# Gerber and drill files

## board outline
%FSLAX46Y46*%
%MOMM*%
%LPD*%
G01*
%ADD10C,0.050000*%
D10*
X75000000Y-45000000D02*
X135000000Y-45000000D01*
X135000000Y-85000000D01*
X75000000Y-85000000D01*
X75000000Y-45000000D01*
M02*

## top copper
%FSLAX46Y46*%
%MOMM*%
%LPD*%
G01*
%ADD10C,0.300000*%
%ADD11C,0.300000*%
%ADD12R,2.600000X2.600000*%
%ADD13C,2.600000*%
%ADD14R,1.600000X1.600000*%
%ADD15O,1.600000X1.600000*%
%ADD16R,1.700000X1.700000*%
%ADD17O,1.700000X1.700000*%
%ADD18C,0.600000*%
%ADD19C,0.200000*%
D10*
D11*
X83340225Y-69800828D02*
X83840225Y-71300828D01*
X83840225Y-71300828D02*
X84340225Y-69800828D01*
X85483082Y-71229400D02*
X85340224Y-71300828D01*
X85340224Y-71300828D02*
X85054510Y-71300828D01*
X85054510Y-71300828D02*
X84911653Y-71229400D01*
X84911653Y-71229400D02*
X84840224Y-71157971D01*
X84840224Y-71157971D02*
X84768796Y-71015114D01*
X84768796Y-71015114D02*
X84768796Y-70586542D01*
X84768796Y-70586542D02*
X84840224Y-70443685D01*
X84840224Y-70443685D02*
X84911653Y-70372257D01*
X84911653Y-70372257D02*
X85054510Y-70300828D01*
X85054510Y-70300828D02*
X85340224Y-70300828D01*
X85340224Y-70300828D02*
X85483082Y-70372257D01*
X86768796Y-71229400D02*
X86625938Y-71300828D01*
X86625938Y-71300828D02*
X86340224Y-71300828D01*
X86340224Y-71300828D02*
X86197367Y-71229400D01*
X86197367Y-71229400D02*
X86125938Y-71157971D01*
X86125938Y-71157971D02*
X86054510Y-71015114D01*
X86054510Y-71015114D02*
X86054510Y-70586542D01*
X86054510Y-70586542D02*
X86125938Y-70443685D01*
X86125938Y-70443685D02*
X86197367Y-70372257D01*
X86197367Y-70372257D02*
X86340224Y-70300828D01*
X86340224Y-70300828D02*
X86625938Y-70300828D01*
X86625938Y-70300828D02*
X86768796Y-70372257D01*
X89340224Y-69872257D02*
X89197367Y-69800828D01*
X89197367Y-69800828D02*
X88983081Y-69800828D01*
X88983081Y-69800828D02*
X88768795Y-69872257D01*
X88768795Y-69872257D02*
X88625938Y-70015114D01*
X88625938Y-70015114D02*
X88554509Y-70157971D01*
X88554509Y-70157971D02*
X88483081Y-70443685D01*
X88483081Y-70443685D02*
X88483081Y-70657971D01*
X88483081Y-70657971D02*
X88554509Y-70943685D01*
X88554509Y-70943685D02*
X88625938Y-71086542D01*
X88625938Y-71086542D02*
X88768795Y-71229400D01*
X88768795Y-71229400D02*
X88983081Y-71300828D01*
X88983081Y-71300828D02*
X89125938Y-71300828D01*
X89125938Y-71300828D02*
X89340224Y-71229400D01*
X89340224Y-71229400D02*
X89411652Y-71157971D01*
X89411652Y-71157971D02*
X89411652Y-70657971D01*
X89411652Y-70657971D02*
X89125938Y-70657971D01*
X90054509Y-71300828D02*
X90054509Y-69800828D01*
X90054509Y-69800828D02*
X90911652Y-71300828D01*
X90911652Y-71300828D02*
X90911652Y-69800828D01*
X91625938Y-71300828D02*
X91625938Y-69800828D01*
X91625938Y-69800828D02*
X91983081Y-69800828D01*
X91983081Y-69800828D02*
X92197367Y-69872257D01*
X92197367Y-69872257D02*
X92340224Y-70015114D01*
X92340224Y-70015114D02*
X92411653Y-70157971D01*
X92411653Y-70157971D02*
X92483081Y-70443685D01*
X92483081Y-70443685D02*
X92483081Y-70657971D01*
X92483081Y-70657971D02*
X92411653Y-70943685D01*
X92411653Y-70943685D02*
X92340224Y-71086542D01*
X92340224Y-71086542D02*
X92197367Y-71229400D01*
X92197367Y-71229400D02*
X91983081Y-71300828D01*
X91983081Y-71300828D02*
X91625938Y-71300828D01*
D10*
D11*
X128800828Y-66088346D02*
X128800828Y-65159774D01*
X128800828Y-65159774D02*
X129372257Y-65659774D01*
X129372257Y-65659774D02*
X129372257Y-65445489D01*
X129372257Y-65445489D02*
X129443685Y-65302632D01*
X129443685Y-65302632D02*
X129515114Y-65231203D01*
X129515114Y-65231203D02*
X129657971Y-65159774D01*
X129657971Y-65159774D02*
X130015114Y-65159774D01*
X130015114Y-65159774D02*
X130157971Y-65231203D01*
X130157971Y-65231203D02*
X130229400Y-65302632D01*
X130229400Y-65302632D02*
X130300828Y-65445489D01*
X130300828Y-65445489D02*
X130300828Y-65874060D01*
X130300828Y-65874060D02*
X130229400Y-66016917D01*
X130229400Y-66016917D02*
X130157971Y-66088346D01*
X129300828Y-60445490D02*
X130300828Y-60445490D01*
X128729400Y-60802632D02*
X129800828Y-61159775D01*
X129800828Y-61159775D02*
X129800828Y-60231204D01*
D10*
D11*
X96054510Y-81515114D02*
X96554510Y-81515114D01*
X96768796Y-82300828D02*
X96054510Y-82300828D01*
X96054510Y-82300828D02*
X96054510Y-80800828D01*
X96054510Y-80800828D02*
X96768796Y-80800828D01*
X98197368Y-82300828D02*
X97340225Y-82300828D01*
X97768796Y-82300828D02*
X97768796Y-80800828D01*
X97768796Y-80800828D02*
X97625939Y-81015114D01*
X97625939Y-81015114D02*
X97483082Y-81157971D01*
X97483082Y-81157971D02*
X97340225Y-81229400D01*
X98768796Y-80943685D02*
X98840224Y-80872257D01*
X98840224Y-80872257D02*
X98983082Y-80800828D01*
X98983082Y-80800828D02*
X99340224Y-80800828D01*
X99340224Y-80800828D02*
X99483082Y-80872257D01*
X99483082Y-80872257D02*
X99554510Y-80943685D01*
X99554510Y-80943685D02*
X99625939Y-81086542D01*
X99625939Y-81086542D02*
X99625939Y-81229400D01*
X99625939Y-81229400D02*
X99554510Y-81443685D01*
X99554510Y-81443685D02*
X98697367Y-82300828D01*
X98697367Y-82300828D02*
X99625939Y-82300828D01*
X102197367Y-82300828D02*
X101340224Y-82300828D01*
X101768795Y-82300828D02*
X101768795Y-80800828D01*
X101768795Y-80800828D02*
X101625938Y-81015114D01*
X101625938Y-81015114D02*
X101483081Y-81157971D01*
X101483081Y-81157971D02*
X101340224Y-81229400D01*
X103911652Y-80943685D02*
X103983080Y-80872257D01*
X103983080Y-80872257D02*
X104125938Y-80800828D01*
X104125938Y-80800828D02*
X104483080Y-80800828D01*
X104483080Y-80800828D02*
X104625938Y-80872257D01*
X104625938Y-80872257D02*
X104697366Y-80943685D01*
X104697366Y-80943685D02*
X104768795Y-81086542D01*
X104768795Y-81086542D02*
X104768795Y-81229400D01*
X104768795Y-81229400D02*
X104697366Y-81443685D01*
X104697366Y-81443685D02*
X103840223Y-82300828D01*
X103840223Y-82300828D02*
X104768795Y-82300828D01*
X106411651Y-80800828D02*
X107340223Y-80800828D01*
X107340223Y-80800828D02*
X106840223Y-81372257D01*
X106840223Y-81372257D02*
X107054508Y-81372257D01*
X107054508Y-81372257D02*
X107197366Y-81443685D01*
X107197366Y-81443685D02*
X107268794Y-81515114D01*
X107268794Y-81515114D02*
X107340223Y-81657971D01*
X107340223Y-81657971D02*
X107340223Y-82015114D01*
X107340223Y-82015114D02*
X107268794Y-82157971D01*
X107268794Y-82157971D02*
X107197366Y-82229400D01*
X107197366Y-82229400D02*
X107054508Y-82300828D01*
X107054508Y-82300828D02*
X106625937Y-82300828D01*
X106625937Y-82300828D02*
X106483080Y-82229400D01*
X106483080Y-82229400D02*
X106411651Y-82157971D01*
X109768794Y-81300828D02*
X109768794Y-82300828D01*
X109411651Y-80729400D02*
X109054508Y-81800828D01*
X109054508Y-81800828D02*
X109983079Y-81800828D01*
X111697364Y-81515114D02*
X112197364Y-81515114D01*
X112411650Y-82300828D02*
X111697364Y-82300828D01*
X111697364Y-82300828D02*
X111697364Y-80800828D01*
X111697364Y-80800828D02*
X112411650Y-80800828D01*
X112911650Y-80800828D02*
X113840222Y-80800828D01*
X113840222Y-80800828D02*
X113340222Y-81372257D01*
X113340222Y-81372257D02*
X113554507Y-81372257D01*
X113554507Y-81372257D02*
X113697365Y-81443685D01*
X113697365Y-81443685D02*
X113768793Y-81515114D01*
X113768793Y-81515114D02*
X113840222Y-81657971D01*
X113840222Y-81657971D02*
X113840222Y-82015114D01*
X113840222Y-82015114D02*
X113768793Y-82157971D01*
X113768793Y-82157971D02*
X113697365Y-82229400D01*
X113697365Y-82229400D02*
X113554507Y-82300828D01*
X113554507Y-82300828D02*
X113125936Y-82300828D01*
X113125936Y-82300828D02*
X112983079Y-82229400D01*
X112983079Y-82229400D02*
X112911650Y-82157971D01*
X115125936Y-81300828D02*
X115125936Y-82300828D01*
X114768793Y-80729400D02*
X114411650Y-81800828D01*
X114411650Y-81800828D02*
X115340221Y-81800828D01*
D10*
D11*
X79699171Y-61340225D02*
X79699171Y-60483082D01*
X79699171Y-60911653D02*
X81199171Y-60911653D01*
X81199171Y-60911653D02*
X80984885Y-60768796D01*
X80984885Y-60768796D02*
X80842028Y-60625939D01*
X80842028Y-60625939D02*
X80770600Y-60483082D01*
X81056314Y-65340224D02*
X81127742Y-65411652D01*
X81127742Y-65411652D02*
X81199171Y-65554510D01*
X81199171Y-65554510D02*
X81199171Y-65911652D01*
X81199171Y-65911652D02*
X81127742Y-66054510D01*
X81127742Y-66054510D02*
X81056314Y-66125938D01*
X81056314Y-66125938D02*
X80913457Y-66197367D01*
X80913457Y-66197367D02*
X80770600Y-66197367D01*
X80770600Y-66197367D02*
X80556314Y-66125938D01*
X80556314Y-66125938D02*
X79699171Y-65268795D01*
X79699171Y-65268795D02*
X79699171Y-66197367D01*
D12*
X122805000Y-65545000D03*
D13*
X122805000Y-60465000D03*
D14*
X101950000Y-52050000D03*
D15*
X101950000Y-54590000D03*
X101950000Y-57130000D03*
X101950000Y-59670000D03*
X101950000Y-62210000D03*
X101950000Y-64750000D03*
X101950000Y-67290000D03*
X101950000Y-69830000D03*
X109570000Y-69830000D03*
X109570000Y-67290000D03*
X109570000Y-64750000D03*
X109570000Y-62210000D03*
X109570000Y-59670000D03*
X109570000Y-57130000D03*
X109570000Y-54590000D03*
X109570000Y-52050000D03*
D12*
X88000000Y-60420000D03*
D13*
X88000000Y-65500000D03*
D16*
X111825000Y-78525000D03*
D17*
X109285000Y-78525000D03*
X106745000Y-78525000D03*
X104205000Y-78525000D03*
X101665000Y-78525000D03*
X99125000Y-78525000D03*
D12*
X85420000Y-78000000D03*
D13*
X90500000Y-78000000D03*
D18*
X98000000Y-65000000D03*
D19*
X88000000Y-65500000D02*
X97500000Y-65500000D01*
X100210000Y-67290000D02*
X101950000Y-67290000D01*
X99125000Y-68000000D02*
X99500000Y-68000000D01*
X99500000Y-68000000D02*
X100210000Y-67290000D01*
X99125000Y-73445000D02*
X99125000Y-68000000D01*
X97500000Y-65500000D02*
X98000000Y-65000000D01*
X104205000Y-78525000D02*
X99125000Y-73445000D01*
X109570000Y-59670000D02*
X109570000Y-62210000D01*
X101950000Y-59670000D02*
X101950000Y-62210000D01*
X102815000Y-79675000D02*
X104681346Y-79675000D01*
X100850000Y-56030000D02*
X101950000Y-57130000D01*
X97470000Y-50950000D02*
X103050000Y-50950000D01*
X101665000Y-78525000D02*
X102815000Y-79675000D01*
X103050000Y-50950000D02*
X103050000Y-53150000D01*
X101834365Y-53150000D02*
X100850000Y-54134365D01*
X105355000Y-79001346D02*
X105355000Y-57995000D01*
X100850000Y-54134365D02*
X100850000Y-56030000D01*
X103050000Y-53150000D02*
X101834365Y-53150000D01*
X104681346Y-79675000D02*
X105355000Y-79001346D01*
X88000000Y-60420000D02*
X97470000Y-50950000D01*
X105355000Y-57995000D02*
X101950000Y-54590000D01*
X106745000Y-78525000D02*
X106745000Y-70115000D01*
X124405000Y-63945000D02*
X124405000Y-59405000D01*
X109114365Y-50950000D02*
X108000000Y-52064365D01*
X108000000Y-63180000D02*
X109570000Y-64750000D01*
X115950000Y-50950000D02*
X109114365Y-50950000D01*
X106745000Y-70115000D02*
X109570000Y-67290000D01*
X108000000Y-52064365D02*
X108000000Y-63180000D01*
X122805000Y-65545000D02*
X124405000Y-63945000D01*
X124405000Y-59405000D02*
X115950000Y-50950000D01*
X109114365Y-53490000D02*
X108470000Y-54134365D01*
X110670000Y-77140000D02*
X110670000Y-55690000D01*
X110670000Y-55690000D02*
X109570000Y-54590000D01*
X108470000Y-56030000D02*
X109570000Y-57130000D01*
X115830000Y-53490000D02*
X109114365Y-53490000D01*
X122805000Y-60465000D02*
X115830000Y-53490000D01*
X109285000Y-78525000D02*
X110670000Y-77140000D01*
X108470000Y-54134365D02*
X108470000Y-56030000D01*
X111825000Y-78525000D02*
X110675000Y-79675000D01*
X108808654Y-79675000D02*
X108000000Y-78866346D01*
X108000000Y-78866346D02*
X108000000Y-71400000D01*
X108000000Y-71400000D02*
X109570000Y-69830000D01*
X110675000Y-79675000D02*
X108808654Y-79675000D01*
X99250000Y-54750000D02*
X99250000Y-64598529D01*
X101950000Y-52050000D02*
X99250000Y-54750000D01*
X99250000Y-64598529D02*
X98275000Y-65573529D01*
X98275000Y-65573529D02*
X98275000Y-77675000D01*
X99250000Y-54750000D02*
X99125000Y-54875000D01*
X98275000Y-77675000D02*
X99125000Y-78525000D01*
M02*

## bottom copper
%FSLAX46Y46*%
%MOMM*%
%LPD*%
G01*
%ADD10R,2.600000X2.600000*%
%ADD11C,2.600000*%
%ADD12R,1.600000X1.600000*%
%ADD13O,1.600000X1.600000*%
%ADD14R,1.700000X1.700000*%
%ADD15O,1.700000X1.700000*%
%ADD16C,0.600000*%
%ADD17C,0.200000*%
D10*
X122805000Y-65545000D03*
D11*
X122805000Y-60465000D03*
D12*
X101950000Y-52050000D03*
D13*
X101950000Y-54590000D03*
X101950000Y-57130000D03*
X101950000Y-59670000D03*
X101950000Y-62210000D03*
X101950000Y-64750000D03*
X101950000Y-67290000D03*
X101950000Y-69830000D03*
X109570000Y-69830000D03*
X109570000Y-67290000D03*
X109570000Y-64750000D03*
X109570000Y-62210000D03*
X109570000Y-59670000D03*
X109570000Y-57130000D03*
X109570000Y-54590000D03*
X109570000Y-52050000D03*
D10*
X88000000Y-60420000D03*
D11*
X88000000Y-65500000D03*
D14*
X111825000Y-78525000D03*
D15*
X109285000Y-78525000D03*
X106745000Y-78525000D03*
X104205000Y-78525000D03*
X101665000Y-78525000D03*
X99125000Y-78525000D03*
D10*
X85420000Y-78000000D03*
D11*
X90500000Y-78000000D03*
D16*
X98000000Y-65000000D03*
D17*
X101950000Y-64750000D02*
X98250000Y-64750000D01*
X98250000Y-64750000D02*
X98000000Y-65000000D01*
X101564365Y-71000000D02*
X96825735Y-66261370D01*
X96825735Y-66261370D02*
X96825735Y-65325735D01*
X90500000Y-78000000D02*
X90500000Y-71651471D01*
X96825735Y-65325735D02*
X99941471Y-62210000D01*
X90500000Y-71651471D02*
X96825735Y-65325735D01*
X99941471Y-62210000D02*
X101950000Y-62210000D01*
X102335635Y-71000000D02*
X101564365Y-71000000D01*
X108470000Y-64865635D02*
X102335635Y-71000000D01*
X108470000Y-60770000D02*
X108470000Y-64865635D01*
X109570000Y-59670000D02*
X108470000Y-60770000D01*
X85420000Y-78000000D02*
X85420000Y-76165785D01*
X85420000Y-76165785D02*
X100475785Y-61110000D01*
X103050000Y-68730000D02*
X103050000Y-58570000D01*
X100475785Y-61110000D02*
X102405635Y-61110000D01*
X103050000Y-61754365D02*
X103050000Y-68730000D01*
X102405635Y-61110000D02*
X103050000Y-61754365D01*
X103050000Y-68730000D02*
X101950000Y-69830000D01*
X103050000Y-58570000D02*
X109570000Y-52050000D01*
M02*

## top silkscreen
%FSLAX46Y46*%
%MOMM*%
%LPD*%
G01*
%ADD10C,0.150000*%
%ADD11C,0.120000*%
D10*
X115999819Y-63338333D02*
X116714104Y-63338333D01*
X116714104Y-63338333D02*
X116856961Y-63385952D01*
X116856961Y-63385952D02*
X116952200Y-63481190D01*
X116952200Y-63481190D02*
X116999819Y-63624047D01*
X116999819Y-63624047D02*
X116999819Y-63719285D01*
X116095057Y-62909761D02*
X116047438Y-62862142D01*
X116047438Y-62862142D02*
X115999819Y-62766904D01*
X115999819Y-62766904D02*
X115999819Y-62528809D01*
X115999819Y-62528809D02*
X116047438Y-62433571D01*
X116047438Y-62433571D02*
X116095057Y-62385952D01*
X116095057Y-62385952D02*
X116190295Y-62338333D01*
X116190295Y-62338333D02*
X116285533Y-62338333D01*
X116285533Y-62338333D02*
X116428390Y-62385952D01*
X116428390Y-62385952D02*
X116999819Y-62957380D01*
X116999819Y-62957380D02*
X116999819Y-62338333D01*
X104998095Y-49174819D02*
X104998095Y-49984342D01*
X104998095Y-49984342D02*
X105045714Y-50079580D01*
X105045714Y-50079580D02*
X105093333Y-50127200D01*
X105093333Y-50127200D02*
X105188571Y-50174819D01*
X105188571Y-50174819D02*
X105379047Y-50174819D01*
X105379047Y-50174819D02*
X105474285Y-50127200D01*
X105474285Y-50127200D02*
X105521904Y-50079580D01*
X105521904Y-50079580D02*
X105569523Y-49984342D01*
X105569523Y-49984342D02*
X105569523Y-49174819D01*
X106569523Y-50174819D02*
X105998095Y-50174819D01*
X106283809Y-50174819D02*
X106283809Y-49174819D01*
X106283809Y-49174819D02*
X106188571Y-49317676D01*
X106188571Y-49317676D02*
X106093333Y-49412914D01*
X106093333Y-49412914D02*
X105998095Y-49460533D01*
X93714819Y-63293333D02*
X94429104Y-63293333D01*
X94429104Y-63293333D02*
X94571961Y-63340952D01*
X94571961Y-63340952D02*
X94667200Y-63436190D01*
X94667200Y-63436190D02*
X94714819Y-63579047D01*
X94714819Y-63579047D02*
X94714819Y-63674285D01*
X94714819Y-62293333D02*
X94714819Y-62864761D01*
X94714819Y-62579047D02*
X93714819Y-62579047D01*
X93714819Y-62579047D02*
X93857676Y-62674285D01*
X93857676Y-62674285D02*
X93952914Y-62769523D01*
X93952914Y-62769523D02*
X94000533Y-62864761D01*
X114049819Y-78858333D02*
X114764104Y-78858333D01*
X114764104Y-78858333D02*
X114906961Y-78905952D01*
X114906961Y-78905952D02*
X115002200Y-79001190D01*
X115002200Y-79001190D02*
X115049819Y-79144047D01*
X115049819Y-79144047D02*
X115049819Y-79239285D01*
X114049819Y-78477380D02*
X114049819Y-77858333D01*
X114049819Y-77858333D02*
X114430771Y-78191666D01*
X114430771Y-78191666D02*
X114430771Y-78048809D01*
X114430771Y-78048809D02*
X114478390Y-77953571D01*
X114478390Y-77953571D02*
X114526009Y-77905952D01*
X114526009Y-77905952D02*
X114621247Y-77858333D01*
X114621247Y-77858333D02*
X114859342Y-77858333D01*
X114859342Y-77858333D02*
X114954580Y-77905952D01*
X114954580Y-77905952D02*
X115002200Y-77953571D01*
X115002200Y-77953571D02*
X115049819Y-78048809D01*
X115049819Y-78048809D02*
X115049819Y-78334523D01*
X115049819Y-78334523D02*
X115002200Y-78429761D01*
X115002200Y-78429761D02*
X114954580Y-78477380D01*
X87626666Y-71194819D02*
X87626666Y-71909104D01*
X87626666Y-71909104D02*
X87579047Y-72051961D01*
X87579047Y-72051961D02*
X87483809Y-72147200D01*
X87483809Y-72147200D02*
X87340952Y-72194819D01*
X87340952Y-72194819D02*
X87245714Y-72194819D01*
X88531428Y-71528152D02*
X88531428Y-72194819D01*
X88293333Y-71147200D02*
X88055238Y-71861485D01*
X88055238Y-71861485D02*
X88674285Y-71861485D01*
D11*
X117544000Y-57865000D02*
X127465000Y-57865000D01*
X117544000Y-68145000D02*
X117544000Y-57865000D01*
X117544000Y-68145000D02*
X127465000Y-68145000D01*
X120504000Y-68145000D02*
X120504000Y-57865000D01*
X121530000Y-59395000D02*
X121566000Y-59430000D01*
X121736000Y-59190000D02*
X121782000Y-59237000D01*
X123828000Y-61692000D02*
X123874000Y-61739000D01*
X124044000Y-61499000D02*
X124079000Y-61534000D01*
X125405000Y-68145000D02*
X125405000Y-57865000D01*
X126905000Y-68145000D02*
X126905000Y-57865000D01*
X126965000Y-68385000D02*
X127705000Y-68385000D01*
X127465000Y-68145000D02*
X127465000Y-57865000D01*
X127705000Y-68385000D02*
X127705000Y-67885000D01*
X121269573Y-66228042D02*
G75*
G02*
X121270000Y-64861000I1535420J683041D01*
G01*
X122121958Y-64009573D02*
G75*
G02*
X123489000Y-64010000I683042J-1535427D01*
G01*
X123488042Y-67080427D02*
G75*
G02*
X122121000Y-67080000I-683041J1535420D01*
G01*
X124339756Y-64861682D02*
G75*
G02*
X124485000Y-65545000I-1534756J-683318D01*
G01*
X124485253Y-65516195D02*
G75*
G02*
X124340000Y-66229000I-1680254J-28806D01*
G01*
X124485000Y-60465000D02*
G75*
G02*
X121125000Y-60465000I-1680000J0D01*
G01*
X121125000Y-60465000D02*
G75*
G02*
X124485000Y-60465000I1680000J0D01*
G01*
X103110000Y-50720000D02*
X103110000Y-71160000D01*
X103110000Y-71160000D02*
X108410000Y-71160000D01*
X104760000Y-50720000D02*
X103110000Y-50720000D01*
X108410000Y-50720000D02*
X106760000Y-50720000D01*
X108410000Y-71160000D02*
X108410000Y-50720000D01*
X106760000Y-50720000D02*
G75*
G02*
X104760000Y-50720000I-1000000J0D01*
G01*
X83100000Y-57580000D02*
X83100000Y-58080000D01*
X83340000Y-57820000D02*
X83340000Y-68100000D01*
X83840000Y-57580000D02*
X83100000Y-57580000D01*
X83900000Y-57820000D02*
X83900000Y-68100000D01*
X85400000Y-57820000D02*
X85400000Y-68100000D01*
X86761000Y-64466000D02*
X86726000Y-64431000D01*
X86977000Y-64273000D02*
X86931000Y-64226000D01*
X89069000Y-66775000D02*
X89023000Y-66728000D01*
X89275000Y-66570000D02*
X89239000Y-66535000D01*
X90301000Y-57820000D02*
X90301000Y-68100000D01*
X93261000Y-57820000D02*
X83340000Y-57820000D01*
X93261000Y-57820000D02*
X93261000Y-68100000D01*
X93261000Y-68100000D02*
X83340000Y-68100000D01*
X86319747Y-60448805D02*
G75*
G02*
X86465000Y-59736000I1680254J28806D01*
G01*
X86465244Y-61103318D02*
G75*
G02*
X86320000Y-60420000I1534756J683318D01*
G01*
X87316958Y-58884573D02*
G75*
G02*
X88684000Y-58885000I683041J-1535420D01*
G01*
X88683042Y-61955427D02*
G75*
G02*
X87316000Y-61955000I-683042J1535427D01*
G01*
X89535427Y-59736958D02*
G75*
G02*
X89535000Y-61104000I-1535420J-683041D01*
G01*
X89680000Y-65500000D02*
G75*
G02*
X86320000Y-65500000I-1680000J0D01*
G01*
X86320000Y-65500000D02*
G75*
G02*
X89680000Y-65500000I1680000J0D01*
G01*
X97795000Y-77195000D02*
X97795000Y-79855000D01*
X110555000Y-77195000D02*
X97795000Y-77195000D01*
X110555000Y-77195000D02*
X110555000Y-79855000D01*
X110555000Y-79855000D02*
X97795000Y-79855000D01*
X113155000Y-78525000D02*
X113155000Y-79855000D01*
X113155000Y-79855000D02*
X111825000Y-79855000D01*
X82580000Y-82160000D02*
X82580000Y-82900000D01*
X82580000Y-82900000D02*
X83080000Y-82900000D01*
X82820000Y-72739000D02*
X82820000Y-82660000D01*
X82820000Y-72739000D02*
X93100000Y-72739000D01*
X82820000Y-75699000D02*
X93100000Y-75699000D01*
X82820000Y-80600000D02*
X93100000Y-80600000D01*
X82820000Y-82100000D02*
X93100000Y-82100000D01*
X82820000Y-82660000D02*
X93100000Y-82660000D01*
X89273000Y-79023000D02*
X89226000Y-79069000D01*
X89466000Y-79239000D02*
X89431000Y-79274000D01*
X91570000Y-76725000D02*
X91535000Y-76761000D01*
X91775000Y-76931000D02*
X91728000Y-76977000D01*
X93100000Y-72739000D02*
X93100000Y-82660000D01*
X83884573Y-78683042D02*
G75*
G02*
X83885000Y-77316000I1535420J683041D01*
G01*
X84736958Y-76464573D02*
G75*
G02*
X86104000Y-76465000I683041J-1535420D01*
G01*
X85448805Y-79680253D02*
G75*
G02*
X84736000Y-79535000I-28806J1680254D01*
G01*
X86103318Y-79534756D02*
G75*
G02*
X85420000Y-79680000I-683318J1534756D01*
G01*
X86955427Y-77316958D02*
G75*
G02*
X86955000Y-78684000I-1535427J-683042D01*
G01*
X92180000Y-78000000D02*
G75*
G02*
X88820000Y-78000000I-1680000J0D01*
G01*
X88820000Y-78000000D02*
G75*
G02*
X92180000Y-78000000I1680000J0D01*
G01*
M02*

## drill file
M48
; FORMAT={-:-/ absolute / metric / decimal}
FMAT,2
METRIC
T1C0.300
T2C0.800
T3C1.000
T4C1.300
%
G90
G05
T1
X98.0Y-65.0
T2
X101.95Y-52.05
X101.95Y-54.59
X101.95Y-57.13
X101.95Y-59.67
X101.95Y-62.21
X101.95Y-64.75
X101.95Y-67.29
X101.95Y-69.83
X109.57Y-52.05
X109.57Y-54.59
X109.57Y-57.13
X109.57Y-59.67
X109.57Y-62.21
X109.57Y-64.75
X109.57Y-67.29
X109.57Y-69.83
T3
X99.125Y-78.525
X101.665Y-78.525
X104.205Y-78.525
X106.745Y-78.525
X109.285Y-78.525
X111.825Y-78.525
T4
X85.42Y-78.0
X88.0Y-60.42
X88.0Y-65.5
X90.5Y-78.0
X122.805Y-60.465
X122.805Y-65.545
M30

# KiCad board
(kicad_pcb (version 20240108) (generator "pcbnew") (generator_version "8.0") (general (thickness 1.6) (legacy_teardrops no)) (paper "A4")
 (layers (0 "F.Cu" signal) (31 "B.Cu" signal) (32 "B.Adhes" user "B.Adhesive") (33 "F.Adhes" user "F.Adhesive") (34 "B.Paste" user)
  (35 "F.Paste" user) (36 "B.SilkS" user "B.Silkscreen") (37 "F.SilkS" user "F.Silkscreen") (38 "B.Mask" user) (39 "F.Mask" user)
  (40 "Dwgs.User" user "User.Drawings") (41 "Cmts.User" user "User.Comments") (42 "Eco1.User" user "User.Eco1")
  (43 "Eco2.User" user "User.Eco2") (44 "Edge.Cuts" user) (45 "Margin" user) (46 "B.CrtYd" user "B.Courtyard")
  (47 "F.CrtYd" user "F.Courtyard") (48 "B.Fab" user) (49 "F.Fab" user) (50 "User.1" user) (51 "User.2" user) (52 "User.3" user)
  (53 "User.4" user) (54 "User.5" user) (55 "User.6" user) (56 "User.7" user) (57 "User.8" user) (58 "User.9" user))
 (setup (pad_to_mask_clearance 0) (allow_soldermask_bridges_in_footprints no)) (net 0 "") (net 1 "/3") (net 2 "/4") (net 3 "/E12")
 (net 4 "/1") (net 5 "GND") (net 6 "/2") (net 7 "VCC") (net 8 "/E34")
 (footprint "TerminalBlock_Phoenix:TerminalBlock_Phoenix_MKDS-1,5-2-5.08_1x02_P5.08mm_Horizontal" (layer "F.Cu") (at 122.805 65.545 90)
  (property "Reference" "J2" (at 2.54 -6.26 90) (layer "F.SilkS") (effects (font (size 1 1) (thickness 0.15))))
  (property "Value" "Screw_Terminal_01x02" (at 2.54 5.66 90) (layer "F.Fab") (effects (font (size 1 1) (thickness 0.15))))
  (fp_line (start 7.68 -5.261) (end 7.68 4.66) (stroke (width 0.12) (type solid)) (layer "F.SilkS"))
  (fp_line (start -2.6 -5.261) (end 7.68 -5.261) (stroke (width 0.12) (type solid)) (layer "F.SilkS"))
  (fp_line (start -2.6 -5.261) (end -2.6 4.66) (stroke (width 0.12) (type solid)) (layer "F.SilkS"))
  (fp_line (start -2.6 -2.301) (end 7.68 -2.301) (stroke (width 0.12) (type solid)) (layer "F.SilkS"))
  (fp_line (start 6.15 -1.275) (end 6.115 -1.239) (stroke (width 0.12) (type solid)) (layer "F.SilkS"))
  (fp_line (start 6.355 -1.069) (end 6.308 -1.023) (stroke (width 0.12) (type solid)) (layer "F.SilkS"))
  (fp_line (start 3.853 1.023) (end 3.806 1.069) (stroke (width 0.12) (type solid)) (layer "F.SilkS"))
  (fp_line (start 4.046 1.239) (end 4.011 1.274) (stroke (width 0.12) (type solid)) (layer "F.SilkS"))
  (fp_line (start -2.6 2.6) (end 7.68 2.6) (stroke (width 0.12) (type solid)) (layer "F.SilkS"))
  (fp_line (start -2.6 4.1) (end 7.68 4.1) (stroke (width 0.12) (type solid)) (layer "F.SilkS"))
  (fp_line (start -2.84 4.16) (end -2.84 4.9) (stroke (width 0.12) (type solid)) (layer "F.SilkS"))
  (fp_line (start -2.6 4.66) (end 7.68 4.66) (stroke (width 0.12) (type solid)) (layer "F.SilkS"))
  (fp_line (start -2.84 4.9) (end -2.34 4.9) (stroke (width 0.12) (type solid)) (layer "F.SilkS"))
  (fp_arc (start -0.683042 -1.535427) (mid 0.000524 -1.680501) (end 0.684 -1.535) (stroke (width 0.12) (type solid)) (layer "F.SilkS"))
  (fp_arc (start 1.535427 -0.683042) (mid 1.680501 0.000524) (end 1.535 0.684) (stroke (width 0.12) (type solid)) (layer "F.SilkS"))
  (fp_arc (start -1.535427 0.683042) (mid -1.680501 -0.000524) (end -1.535 -0.684) (stroke (width 0.12) (type solid)) (layer "F.SilkS"))
  (fp_arc (start 0.683318 1.534756) (mid 0.349292 1.643288) (end 0 1.68) (stroke (width 0.12) (type solid)) (layer "F.SilkS"))
  (fp_arc (start 0.028805 1.680253) (mid -0.335551 1.646659) (end -0.684 1.535) (stroke (width 0.12) (type solid)) (layer "F.SilkS"))
  (fp_circle (center 5.08 0) (end 6.76 0) (stroke (width 0.12) (type solid)) (fill none) (layer "F.SilkS"))
  (pad "1" thru_hole rect (at 0 0 90) (size 2.6 2.6) (drill 1.3) (layers "*.Cu" "*.Mask") (remove_unused_layers no) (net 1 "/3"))
  (pad "2" thru_hole circle (at 5.08 0 90) (size 2.6 2.6) (drill 1.3) (layers "*.Cu" "*.Mask") (remove_unused_layers no) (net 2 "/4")))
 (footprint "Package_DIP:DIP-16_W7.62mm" (layer "F.Cu") (at 101.95 52.05)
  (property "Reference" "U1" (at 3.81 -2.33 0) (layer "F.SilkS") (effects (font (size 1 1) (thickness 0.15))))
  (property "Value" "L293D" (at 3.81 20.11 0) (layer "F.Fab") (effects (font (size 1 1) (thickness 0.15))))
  (fp_line (start 1.16 -1.33) (end 1.16 19.11) (stroke (width 0.12) (type solid)) (layer "F.SilkS"))
  (fp_line (start 1.16 19.11) (end 6.46 19.11) (stroke (width 0.12) (type solid)) (layer "F.SilkS"))
  (fp_line (start 2.81 -1.33) (end 1.16 -1.33) (stroke (width 0.12) (type solid)) (layer "F.SilkS"))
  (fp_line (start 6.46 -1.33) (end 4.81 -1.33) (stroke (width 0.12) (type solid)) (layer "F.SilkS"))
  (fp_line (start 6.46 19.11) (end 6.46 -1.33) (stroke (width 0.12) (type solid)) (layer "F.SilkS"))
  (fp_arc (start 4.81 -1.33) (mid 3.81 -0.33) (end 2.81 -1.33) (stroke (width 0.12) (type solid)) (layer "F.SilkS"))
  (pad "1" thru_hole rect (at 0 0) (size 1.6 1.6) (drill 0.8) (layers "*.Cu" "*.Mask") (remove_unused_layers no) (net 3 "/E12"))
  (pad "2" thru_hole oval (at 0 2.54) (size 1.6 1.6) (drill 0.8) (layers "*.Cu" "*.Mask") (remove_unused_layers no) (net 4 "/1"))
  (pad "3" thru_hole oval (at 0 5.08) (size 1.6 1.6) (drill 0.8) (layers "*.Cu" "*.Mask") (remove_unused_layers no) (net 4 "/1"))
  (pad "4" thru_hole oval (at 0 7.62) (size 1.6 1.6) (drill 0.8) (layers "*.Cu" "*.Mask") (remove_unused_layers no) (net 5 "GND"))
  (pad "5" thru_hole oval (at 0 10.16) (size 1.6 1.6) (drill 0.8) (layers "*.Cu" "*.Mask") (remove_unused_layers no) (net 5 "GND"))
  (pad "6" thru_hole oval (at 0 12.7) (size 1.6 1.6) (drill 0.8) (layers "*.Cu" "*.Mask") (remove_unused_layers no) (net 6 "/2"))
  (pad "7" thru_hole oval (at 0 15.24) (size 1.6 1.6) (drill 0.8) (layers "*.Cu" "*.Mask") (remove_unused_layers no) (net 6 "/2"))
  (pad "8" thru_hole oval (at 0 17.78) (size 1.6 1.6) (drill 0.8) (layers "*.Cu" "*.Mask") (remove_unused_layers no) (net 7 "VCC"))
  (pad "9" thru_hole oval (at 7.62 17.78) (size 1.6 1.6) (drill 0.8) (layers "*.Cu" "*.Mask") (remove_unused_layers no) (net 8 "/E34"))
  (pad "10" thru_hole oval (at 7.62 15.24) (size 1.6 1.6) (drill 0.8) (layers "*.Cu" "*.Mask") (remove_unused_layers no) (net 1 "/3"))
  (pad "11" thru_hole oval (at 7.62 12.7) (size 1.6 1.6) (drill 0.8) (layers "*.Cu" "*.Mask") (remove_unused_layers no) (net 1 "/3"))
  (pad "12" thru_hole oval (at 7.62 10.16) (size 1.6 1.6) (drill 0.8) (layers "*.Cu" "*.Mask") (remove_unused_layers no) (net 5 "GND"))
  (pad "13" thru_hole oval (at 7.62 7.62) (size 1.6 1.6) (drill 0.8) (layers "*.Cu" "*.Mask") (remove_unused_layers no) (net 5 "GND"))
  (pad "14" thru_hole oval (at 7.62 5.08) (size 1.6 1.6) (drill 0.8) (layers "*.Cu" "*.Mask") (remove_unused_layers no) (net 2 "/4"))
  (pad "15" thru_hole oval (at 7.62 2.54) (size 1.6 1.6) (drill 0.8) (layers "*.Cu" "*.Mask") (remove_unused_layers no) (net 2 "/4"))
  (pad "16" thru_hole oval (at 7.62 0) (size 1.6 1.6) (drill 0.8) (layers "*.Cu" "*.Mask") (remove_unused_layers no) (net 7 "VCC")))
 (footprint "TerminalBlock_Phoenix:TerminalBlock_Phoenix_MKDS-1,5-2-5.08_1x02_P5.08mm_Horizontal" (layer "F.Cu") (at 88 60.42 -90)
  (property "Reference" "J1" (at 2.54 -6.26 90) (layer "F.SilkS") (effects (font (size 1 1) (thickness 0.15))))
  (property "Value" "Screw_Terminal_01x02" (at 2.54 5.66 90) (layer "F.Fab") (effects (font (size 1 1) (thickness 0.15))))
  (fp_line (start -2.84 4.9) (end -2.34 4.9) (stroke (width 0.12) (type solid)) (layer "F.SilkS"))
  (fp_line (start -2.6 4.66) (end 7.68 4.66) (stroke (width 0.12) (type solid)) (layer "F.SilkS"))
  (fp_line (start -2.84 4.16) (end -2.84 4.9) (stroke (width 0.12) (type solid)) (layer "F.SilkS"))
  (fp_line (start -2.6 4.1) (end 7.68 4.1) (stroke (width 0.12) (type solid)) (layer "F.SilkS"))
  (fp_line (start -2.6 2.6) (end 7.68 2.6) (stroke (width 0.12) (type solid)) (layer "F.SilkS"))
  (fp_line (start 4.046 1.239) (end 4.011 1.274) (stroke (width 0.12) (type solid)) (layer "F.SilkS"))
  (fp_line (start 3.853 1.023) (end 3.806 1.069) (stroke (width 0.12) (type solid)) (layer "F.SilkS"))
  (fp_line (start 6.355 -1.069) (end 6.308 -1.023) (stroke (width 0.12) (type solid)) (layer "F.SilkS"))
  (fp_line (start 6.15 -1.275) (end 6.115 -1.239) (stroke (width 0.12) (type solid)) (layer "F.SilkS"))
  (fp_line (start -2.6 -2.301) (end 7.68 -2.301) (stroke (width 0.12) (type solid)) (layer "F.SilkS"))
  (fp_line (start -2.6 -5.261) (end -2.6 4.66) (stroke (width 0.12) (type solid)) (layer "F.SilkS"))
  (fp_line (start -2.6 -5.261) (end 7.68 -5.261) (stroke (width 0.12) (type solid)) (layer "F.SilkS"))
  (fp_line (start 7.68 -5.261) (end 7.68 4.66) (stroke (width 0.12) (type solid)) (layer "F.SilkS"))
  (fp_arc (start 0.028805 1.680253) (mid -0.335551 1.646659) (end -0.684 1.535) (stroke (width 0.12) (type solid)) (layer "F.SilkS"))
  (fp_arc (start 0.683318 1.534756) (mid 0.349292 1.643288) (end 0 1.68) (stroke (width 0.12) (type solid)) (layer "F.SilkS"))
  (fp_arc (start -1.535427 0.683042) (mid -1.680501 -0.000524) (end -1.535 -0.684) (stroke (width 0.12) (type solid)) (layer "F.SilkS"))
  (fp_arc (start 1.535427 -0.683042) (mid 1.680501 0.000524) (end 1.535 0.684) (stroke (width 0.12) (type solid)) (layer "F.SilkS"))
  (fp_arc (start -0.683042 -1.535427) (mid 0.000524 -1.680501) (end 0.684 -1.535) (stroke (width 0.12) (type solid)) (layer "F.SilkS"))
  (fp_circle (center 5.08 0) (end 6.76 0) (stroke (width 0.12) (type solid)) (fill none) (layer "F.SilkS"))
  (pad "1" thru_hole rect (at 0 0 270) (size 2.6 2.6) (drill 1.3) (layers "*.Cu" "*.Mask") (remove_unused_layers no) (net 4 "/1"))
  (pad "2" thru_hole circle (at 5.08 0 270) (size 2.6 2.6) (drill 1.3) (layers "*.Cu" "*.Mask") (remove_unused_layers no) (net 6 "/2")))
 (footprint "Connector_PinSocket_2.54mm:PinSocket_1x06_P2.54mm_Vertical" (layer "F.Cu") (at 111.825 78.525 -90)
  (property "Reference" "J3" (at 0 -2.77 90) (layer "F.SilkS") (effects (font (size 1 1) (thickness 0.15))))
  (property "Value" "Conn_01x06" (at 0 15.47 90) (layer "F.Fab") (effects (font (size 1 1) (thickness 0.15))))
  (fp_line (start -1.33 14.03) (end 1.33 14.03) (stroke (width 0.12) (type solid)) (layer "F.SilkS"))
  (fp_line (start -1.33 1.27) (end -1.33 14.03) (stroke (width 0.12) (type solid)) (layer "F.SilkS"))
  (fp_line (start -1.33 1.27) (end 1.33 1.27) (stroke (width 0.12) (type solid)) (layer "F.SilkS"))
  (fp_line (start 1.33 1.27) (end 1.33 14.03) (stroke (width 0.12) (type solid)) (layer "F.SilkS"))
  (fp_line (start 0 -1.33) (end 1.33 -1.33) (stroke (width 0.12) (type solid)) (layer "F.SilkS"))
  (fp_line (start 1.33 -1.33) (end 1.33 0) (stroke (width 0.12) (type solid)) (layer "F.SilkS"))
  (pad "1" thru_hole rect (at 0 0 270) (size 1.7 1.7) (drill 1) (layers "*.Cu" "*.Mask") (remove_unused_layers no) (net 8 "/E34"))
  (pad "2" thru_hole oval (at 0 2.54 270) (size 1.7 1.7) (drill 1) (layers "*.Cu" "*.Mask") (remove_unused_layers no) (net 2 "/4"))
  (pad "3" thru_hole oval (at 0 5.08 270) (size 1.7 1.7) (drill 1) (layers "*.Cu" "*.Mask") (remove_unused_layers no) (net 1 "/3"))
  (pad "4" thru_hole oval (at 0 7.62 270) (size 1.7 1.7) (drill 1) (layers "*.Cu" "*.Mask") (remove_unused_layers no) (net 6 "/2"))
  (pad "5" thru_hole oval (at 0 10.16 270) (size 1.7 1.7) (drill 1) (layers "*.Cu" "*.Mask") (remove_unused_layers no) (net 4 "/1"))
  (pad "6" thru_hole oval (at 0 12.7 270) (size 1.7 1.7) (drill 1) (layers "*.Cu" "*.Mask") (remove_unused_layers no) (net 3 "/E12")))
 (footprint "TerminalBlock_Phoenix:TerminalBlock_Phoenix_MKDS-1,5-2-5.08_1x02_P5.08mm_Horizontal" (layer "F.Cu") (at 85.42 78)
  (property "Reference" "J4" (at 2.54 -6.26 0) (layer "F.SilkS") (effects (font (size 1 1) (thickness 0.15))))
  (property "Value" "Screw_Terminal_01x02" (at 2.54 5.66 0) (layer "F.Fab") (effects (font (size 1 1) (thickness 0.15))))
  (fp_line (start -2.84 4.16) (end -2.84 4.9) (stroke (width 0.12) (type solid)) (layer "F.SilkS"))
  (fp_line (start -2.84 4.9) (end -2.34 4.9) (stroke (width 0.12) (type solid)) (layer "F.SilkS"))
  (fp_line (start -2.6 -5.261) (end -2.6 4.66) (stroke (width 0.12) (type solid)) (layer "F.SilkS"))
  (fp_line (start -2.6 -5.261) (end 7.68 -5.261) (stroke (width 0.12) (type solid)) (layer "F.SilkS"))
  (fp_line (start -2.6 -2.301) (end 7.68 -2.301) (stroke (width 0.12) (type solid)) (layer "F.SilkS"))
  (fp_line (start -2.6 2.6) (end 7.68 2.6) (stroke (width 0.12) (type solid)) (layer "F.SilkS"))
  (fp_line (start -2.6 4.1) (end 7.68 4.1) (stroke (width 0.12) (type solid)) (layer "F.SilkS"))
  (fp_line (start -2.6 4.66) (end 7.68 4.66) (stroke (width 0.12) (type solid)) (layer "F.SilkS"))
  (fp_line (start 3.853 1.023) (end 3.806 1.069) (stroke (width 0.12) (type solid)) (layer "F.SilkS"))
  (fp_line (start 4.046 1.239) (end 4.011 1.274) (stroke (width 0.12) (type solid)) (layer "F.SilkS"))
  (fp_line (start 6.15 -1.275) (end 6.115 -1.239) (stroke (width 0.12) (type solid)) (layer "F.SilkS"))
  (fp_line (start 6.355 -1.069) (end 6.308 -1.023) (stroke (width 0.12) (type solid)) (layer "F.SilkS"))
  (fp_line (start 7.68 -5.261) (end 7.68 4.66) (stroke (width 0.12) (type solid)) (layer "F.SilkS"))
  (fp_arc (start -1.535427 0.683042) (mid -1.680501 -0.000524) (end -1.535 -0.684) (stroke (width 0.12) (type solid)) (layer "F.SilkS"))
  (fp_arc (start -0.683042 -1.535427) (mid 0.000524 -1.680501) (end 0.684 -1.535) (stroke (width 0.12) (type solid)) (layer "F.SilkS"))
  (fp_arc (start 0.028805 1.680253) (mid -0.335551 1.646659) (end -0.684 1.535) (stroke (width 0.12) (type solid)) (layer "F.SilkS"))
  (fp_arc (start 0.683318 1.534756) (mid 0.349292 1.643288) (end 0 1.68) (stroke (width 0.12) (type solid)) (layer "F.SilkS"))
  (fp_arc (start 1.535427 -0.683042) (mid 1.680501 0.000524) (end 1.535 0.684) (stroke (width 0.12) (type solid)) (layer "F.SilkS"))
  (fp_circle (center 5.08 0) (end 6.76 0) (stroke (width 0.12) (type solid)) (fill none) (layer "F.SilkS"))
  (pad "1" thru_hole rect (at 0 0) (size 2.6 2.6) (drill 1.3) (layers "*.Cu" "*.Mask") (remove_unused_layers no) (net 7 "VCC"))
  (pad "2" thru_hole circle (at 5.08 0) (size 2.6 2.6) (drill 1.3) (layers "*.Cu" "*.Mask") (remove_unused_layers no) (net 5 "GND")))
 (gr_rect (start 75 45) (end 135 85) (stroke (width 0.05) (type default)) (fill none) (layer "Edge.Cuts"))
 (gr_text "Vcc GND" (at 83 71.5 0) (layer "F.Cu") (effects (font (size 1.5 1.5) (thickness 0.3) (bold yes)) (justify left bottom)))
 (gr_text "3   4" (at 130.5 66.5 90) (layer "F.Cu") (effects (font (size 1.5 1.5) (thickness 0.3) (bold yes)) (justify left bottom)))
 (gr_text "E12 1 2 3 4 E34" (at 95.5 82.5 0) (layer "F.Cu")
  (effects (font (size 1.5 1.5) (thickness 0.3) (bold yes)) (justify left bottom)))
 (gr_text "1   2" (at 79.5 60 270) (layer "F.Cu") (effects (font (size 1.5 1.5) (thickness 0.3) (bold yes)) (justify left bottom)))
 (segment (start 88 65.5) (end 97.5 65.5) (width 0.2) (layer "F.Cu") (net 6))
 (segment (start 100.21 67.29) (end 101.95 67.29) (width 0.2) (layer "F.Cu") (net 6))
 (segment (start 99.125 68) (end 99.5 68) (width 0.2) (layer "F.Cu") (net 6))
 (segment (start 99.5 68) (end 100.21 67.29) (width 0.2) (layer "F.Cu") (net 6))
 (segment (start 99.125 73.445) (end 99.125 68) (width 0.2) (layer "F.Cu") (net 6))
 (segment (start 97.5 65.5) (end 98 65) (width 0.2) (layer "F.Cu") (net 6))
 (segment (start 104.205 78.525) (end 99.125 73.445) (width 0.2) (layer "F.Cu") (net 6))
 (via (at 98 65) (size 0.6) (drill 0.3) (layers "F.Cu" "B.Cu") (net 6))
 (segment (start 101.95 64.75) (end 98.25 64.75) (width 0.2) (layer "B.Cu") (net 6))
 (segment (start 98.25 64.75) (end 98 65) (width 0.2) (layer "B.Cu") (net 6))
 (segment (start 109.57 59.67) (end 109.57 62.21) (width 0.2) (layer "F.Cu") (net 5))
 (segment (start 101.95 59.67) (end 101.95 62.21) (width 0.2) (layer "F.Cu") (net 5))
 (segment (start 101.564365 71) (end 96.825735 66.26137) (width 0.2) (layer "B.Cu") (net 5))
 (segment (start 96.825735 66.26137) (end 96.825735 65.325735) (width 0.2) (layer "B.Cu") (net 5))
 (segment (start 90.5 78) (end 90.5 71.651471) (width 0.2) (layer "B.Cu") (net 5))
 (segment (start 96.825735 65.325735) (end 99.941471 62.21) (width 0.2) (layer "B.Cu") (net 5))
 (segment (start 90.5 71.651471) (end 96.825735 65.325735) (width 0.2) (layer "B.Cu") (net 5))
 (segment (start 99.941471 62.21) (end 101.95 62.21) (width 0.2) (layer "B.Cu") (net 5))
 (segment (start 102.335635 71) (end 101.564365 71) (width 0.2) (layer "B.Cu") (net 5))
 (segment (start 108.47 64.865635) (end 102.335635 71) (width 0.2) (layer "B.Cu") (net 5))
 (segment (start 108.47 60.77) (end 108.47 64.865635) (width 0.2) (layer "B.Cu") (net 5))
 (segment (start 109.57 59.67) (end 108.47 60.77) (width 0.2) (layer "B.Cu") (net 5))
 (segment (start 85.42 78) (end 85.42 76.165785) (width 0.2) (layer "B.Cu") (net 7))
 (segment (start 85.42 76.165785) (end 100.475785 61.11) (width 0.2) (layer "B.Cu") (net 7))
 (segment (start 103.05 68.73) (end 103.05 58.57) (width 0.2) (layer "B.Cu") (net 7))
 (segment (start 100.475785 61.11) (end 102.405635 61.11) (width 0.2) (layer "B.Cu") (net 7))
 (segment (start 103.05 61.754365) (end 103.05 68.73) (width 0.2) (layer "B.Cu") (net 7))
 (segment (start 102.405635 61.11) (end 103.05 61.754365) (width 0.2) (layer "B.Cu") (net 7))
 (segment (start 103.05 68.73) (end 101.95 69.83) (width 0.2) (layer "B.Cu") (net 7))
 (segment (start 103.05 58.57) (end 109.57 52.05) (width 0.2) (layer "B.Cu") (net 7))
 (segment (start 102.815 79.675) (end 104.681346 79.675) (width 0.2) (layer "F.Cu") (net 4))
 (segment (start 100.85 56.03) (end 101.95 57.13) (width 0.2) (layer "F.Cu") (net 4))
 (segment (start 97.47 50.95) (end 103.05 50.95) (width 0.2) (layer "F.Cu") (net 4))
 (segment (start 101.665 78.525) (end 102.815 79.675) (width 0.2) (layer "F.Cu") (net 4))
 (segment (start 103.05 50.95) (end 103.05 53.15) (width 0.2) (layer "F.Cu") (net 4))
 (segment (start 101.834365 53.15) (end 100.85 54.134365) (width 0.2) (layer "F.Cu") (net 4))
 (segment (start 105.355 79.001346) (end 105.355 57.995) (width 0.2) (layer "F.Cu") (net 4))
 (segment (start 100.85 54.134365) (end 100.85 56.03) (width 0.2) (layer "F.Cu") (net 4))
 (segment (start 103.05 53.15) (end 101.834365 53.15) (width 0.2) (layer "F.Cu") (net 4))
 (segment (start 104.681346 79.675) (end 105.355 79.001346) (width 0.2) (layer "F.Cu") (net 4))
 (segment (start 88 60.42) (end 97.47 50.95) (width 0.2) (layer "F.Cu") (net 4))
 (segment (start 105.355 57.995) (end 101.95 54.59) (width 0.2) (layer "F.Cu") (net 4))
 (segment (start 106.745 78.525) (end 106.745 70.115) (width 0.2) (layer "F.Cu") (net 1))
 (segment (start 124.405 63.945) (end 124.405 59.405) (width 0.2) (layer "F.Cu") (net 1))
 (segment (start 109.114365 50.95) (end 108 52.064365) (width 0.2) (layer "F.Cu") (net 1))
 (segment (start 108 63.18) (end 109.57 64.75) (width 0.2) (layer "F.Cu") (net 1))
 (segment (start 115.95 50.95) (end 109.114365 50.95) (width 0.2) (layer "F.Cu") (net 1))
 (segment (start 106.745 70.115) (end 109.57 67.29) (width 0.2) (layer "F.Cu") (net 1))
 (segment (start 108 52.064365) (end 108 63.18) (width 0.2) (layer "F.Cu") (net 1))
 (segment (start 122.805 65.545) (end 124.405 63.945) (width 0.2) (layer "F.Cu") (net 1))
 (segment (start 124.405 59.405) (end 115.95 50.95) (width 0.2) (layer "F.Cu") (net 1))
 (segment (start 109.114365 53.49) (end 108.47 54.134365) (width 0.2) (layer "F.Cu") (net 2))
 (segment (start 110.67 77.14) (end 110.67 55.69) (width 0.2) (layer "F.Cu") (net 2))
 (segment (start 110.67 55.69) (end 109.57 54.59) (width 0.2) (layer "F.Cu") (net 2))
 (segment (start 108.47 56.03) (end 109.57 57.13) (width 0.2) (layer "F.Cu") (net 2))
 (segment (start 115.83 53.49) (end 109.114365 53.49) (width 0.2) (layer "F.Cu") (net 2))
 (segment (start 122.805 60.465) (end 115.83 53.49) (width 0.2) (layer "F.Cu") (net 2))
 (segment (start 109.285 78.525) (end 110.67 77.14) (width 0.2) (layer "F.Cu") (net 2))
 (segment (start 108.47 54.134365) (end 108.47 56.03) (width 0.2) (layer "F.Cu") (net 2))
 (segment (start 111.825 78.525) (end 110.675 79.675) (width 0.2) (layer "F.Cu") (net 8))
 (segment (start 108.808654 79.675) (end 108 78.866346) (width 0.2) (layer "F.Cu") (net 8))
 (segment (start 108 78.866346) (end 108 71.4) (width 0.2) (layer "F.Cu") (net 8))
 (segment (start 108 71.4) (end 109.57 69.83) (width 0.2) (layer "F.Cu") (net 8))
 (segment (start 110.675 79.675) (end 108.808654 79.675) (width 0.2) (layer "F.Cu") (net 8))
 (segment (start 99.25 54.75) (end 99.25 64.598529) (width 0.2) (layer "F.Cu") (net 3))
 (segment (start 101.95 52.05) (end 99.25 54.75) (width 0.2) (layer "F.Cu") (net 3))
 (segment (start 99.25 64.598529) (end 98.275 65.573529) (width 0.2) (layer "F.Cu") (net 3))
 (segment (start 98.275 65.573529) (end 98.275 77.675) (width 0.2) (layer "F.Cu") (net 3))
 (segment (start 99.25 54.75) (end 99.125 54.875) (width 0.2) (layer "F.Cu") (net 3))
 (segment (start 98.275 77.675) (end 99.125 78.525) (width 0.2) (layer "F.Cu") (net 3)))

